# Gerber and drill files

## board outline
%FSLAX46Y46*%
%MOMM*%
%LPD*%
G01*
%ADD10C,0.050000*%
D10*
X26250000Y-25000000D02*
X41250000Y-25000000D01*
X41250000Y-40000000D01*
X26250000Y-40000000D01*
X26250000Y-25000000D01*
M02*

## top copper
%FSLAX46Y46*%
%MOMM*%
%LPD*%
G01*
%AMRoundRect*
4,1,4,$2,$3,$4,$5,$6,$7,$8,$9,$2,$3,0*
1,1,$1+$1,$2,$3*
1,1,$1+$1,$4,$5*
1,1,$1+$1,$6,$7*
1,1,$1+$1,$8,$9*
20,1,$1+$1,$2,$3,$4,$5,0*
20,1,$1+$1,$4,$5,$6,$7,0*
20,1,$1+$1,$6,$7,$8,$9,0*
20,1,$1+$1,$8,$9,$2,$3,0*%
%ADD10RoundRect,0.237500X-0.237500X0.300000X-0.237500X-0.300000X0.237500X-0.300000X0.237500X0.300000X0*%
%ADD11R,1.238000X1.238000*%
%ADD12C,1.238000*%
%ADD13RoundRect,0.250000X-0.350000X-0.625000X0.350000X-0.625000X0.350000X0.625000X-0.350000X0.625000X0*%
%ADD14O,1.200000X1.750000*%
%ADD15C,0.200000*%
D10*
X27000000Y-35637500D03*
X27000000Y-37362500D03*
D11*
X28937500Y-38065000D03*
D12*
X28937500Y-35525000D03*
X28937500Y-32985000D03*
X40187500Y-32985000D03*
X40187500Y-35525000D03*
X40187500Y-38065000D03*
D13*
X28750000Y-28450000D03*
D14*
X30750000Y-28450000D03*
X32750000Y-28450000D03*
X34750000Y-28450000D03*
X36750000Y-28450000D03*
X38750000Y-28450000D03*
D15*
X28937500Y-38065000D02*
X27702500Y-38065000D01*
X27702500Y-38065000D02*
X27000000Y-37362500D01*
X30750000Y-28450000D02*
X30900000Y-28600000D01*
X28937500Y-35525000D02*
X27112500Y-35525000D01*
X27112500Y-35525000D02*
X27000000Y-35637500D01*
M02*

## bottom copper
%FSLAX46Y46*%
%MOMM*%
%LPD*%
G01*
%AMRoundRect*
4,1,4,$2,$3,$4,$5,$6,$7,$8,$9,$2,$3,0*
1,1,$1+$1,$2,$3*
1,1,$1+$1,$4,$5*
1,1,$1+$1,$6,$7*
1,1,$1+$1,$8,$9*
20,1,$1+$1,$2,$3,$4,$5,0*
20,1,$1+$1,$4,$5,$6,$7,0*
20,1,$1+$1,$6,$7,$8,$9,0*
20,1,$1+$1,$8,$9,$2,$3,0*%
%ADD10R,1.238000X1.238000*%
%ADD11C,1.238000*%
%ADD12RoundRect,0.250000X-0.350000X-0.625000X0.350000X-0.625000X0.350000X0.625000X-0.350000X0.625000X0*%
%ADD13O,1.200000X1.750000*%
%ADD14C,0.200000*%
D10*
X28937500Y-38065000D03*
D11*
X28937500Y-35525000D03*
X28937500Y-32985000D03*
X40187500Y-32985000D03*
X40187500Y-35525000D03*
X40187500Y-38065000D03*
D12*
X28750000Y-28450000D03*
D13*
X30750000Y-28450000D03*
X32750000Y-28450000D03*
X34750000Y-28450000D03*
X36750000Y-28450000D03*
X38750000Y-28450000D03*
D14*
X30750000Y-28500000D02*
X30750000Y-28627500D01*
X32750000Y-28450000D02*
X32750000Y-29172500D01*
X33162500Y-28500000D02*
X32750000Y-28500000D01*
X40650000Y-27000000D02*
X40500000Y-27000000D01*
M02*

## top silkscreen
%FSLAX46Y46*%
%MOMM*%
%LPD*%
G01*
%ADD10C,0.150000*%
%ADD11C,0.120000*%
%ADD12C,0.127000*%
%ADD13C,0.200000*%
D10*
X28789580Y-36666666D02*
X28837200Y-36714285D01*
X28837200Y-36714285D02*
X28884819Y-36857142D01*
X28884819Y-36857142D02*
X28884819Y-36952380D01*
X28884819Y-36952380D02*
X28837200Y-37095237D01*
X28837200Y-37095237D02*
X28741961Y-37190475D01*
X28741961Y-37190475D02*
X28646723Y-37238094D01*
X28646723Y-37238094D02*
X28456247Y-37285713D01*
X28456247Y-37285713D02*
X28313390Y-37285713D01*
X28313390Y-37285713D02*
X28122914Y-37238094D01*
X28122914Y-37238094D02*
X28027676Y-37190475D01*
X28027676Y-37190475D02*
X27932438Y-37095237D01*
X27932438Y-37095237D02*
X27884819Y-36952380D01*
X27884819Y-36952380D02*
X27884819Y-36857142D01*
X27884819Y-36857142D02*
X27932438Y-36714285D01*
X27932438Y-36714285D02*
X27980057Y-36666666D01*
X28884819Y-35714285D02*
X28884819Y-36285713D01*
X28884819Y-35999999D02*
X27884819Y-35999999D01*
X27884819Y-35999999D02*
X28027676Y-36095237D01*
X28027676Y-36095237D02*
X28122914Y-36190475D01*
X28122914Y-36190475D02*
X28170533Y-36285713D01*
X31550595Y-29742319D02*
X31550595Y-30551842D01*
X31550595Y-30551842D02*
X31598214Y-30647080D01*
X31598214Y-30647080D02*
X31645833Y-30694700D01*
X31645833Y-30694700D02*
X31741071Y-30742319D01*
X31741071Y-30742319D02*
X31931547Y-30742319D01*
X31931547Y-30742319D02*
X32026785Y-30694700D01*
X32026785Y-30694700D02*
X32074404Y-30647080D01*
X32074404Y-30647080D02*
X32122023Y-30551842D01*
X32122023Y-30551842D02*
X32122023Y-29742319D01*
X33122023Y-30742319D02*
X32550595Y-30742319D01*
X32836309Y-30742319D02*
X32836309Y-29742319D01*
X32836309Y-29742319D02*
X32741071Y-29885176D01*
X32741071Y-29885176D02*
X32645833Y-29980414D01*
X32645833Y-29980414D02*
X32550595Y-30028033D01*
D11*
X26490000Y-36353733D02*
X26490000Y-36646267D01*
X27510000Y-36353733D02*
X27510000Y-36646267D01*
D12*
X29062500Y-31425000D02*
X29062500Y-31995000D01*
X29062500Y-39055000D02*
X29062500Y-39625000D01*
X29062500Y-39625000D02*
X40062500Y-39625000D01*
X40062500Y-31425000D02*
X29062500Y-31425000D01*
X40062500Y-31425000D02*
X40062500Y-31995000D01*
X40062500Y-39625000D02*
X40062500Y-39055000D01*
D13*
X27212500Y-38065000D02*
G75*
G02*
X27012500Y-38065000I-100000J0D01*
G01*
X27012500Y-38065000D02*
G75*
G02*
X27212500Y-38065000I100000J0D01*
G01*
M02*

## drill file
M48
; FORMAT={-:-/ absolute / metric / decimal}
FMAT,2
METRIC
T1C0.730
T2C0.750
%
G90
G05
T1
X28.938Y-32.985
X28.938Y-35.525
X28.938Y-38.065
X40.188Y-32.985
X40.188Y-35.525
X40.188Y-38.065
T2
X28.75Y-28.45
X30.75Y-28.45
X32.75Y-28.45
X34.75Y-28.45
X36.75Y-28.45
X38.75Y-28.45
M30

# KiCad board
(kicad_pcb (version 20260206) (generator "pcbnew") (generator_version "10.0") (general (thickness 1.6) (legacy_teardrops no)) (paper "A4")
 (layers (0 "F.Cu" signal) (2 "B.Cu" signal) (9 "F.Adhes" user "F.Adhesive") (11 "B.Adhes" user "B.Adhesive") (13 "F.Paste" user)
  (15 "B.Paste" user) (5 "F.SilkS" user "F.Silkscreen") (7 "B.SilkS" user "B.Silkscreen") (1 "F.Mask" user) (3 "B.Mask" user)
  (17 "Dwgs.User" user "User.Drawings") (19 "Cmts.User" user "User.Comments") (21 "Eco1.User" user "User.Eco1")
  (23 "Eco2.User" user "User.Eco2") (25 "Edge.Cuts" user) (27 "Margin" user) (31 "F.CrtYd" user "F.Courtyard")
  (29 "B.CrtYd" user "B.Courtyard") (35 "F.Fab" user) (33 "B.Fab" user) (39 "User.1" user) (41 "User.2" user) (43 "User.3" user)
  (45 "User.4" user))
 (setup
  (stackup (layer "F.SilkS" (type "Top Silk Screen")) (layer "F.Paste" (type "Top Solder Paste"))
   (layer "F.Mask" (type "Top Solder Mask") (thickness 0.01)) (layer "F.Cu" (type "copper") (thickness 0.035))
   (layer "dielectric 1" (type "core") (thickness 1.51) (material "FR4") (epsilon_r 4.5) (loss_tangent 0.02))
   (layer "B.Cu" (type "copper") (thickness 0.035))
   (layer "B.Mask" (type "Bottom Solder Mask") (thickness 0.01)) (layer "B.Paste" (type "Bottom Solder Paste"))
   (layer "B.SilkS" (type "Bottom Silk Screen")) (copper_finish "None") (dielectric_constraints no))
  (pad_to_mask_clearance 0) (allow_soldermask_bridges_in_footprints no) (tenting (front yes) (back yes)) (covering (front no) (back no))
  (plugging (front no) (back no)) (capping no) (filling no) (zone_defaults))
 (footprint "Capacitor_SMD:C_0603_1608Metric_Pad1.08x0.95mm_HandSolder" (layer "F.Cu") (at 27 36.5 -90)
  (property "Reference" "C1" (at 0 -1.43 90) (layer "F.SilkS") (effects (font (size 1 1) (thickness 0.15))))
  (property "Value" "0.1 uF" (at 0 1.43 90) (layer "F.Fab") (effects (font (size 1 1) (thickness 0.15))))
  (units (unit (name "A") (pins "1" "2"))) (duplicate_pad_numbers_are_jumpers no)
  (fp_line (start -0.146267 0.51) (end 0.146267 0.51) (stroke (width 0.12) (type solid)) (layer "F.SilkS"))
  (fp_line (start -0.146267 -0.51) (end 0.146267 -0.51) (stroke (width 0.12) (type solid)) (layer "F.SilkS"))
  (pad "1" smd roundrect (at -0.8625 0 270) (size 1.075 0.95) (layers "F.Cu" "F.Mask" "F.Paste") (roundrect_rratio 0.25)
   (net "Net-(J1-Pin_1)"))
  (pad "2" smd roundrect (at 0.8625 0 270) (size 1.075 0.95) (layers "F.Cu" "F.Mask" "F.Paste") (roundrect_rratio 0.25)
   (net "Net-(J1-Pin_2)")))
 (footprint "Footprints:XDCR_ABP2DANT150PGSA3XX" (layer "F.Cu") (at 34.5625 35.525)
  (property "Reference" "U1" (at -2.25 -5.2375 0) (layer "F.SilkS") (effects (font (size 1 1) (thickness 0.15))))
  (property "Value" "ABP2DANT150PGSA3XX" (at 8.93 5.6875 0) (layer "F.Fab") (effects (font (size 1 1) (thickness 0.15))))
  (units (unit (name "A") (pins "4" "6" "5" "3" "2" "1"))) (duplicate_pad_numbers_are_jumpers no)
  (fp_line (start -5.5 -4.1) (end -5.5 -3.53) (stroke (width 0.127) (type solid)) (layer "F.SilkS"))
  (fp_line (start -5.5 3.53) (end -5.5 4.1) (stroke (width 0.127) (type solid)) (layer "F.SilkS"))
  (fp_line (start -5.5 4.1) (end 5.5 4.1) (stroke (width 0.127) (type solid)) (layer "F.SilkS"))
  (fp_line (start 5.5 -4.1) (end -5.5 -4.1) (stroke (width 0.127) (type solid)) (layer "F.SilkS"))
  (fp_line (start 5.5 -4.1) (end 5.5 -3.53) (stroke (width 0.127) (type solid)) (layer "F.SilkS"))
  (fp_line (start 5.5 4.1) (end 5.5 3.53) (stroke (width 0.127) (type solid)) (layer "F.SilkS"))
  (fp_circle (center -7.45 2.54) (end -7.35 2.54) (stroke (width 0.2) (type solid)) (fill no) (layer "F.SilkS"))
  (pad "1" thru_hole rect (at -5.625 2.54) (size 1.238 1.238) (drill 0.73) (layers "*.Cu" "*.Mask") (remove_unused_layers no)
   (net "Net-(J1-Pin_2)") (solder_mask_margin 0.102))
  (pad "2" thru_hole circle (at -5.625 0) (size 1.238 1.238) (drill 0.73) (layers "*.Cu" "*.Mask") (remove_unused_layers no)
   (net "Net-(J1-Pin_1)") (solder_mask_margin 0.102))
  (pad "3" thru_hole circle (at -5.625 -2.54) (size 1.238 1.238) (drill 0.73) (layers "*.Cu" "*.Mask") (remove_unused_layers no)
   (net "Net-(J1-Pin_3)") (solder_mask_margin 0.102))
  (pad "4" thru_hole circle (at 5.625 -2.54) (size 1.238 1.238) (drill 0.73) (layers "*.Cu" "*.Mask") (remove_unused_layers no)
   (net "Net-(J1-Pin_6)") (solder_mask_margin 0.102))
  (pad "5" thru_hole circle (at 5.625 0) (size 1.238 1.238) (drill 0.73) (layers "*.Cu" "*.Mask") (remove_unused_layers no)
   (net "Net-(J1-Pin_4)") (solder_mask_margin 0.102))
  (pad "6" thru_hole circle (at 5.625 2.54) (size 1.238 1.238) (drill 0.73) (layers "*.Cu" "*.Mask") (remove_unused_layers no)
   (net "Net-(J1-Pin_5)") (solder_mask_margin 0.102)))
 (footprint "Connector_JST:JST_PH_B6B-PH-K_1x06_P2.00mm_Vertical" (layer "B.Cu") (at 28.75 28.45)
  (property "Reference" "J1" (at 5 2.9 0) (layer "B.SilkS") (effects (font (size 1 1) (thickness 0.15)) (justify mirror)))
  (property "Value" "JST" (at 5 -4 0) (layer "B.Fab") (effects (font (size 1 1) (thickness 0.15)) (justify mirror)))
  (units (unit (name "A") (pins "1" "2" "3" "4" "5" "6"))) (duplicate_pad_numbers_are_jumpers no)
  (pad "1" thru_hole roundrect (at 0 0) (size 1.2 1.75) (drill 0.75) (layers "*.Cu" "*.Mask") (remove_unused_layers no)
   (roundrect_rratio 0.208333) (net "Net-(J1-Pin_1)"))
  (pad "2" thru_hole oval (at 2 0) (size 1.2 1.75) (drill 0.75) (layers "*.Cu" "*.Mask") (remove_unused_layers no) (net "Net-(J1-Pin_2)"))
  (pad "3" thru_hole oval (at 4 0) (size 1.2 1.75) (drill 0.75) (layers "*.Cu" "*.Mask") (remove_unused_layers no) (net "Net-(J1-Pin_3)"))
  (pad "4" thru_hole oval (at 6 0) (size 1.2 1.75) (drill 0.75) (layers "*.Cu" "*.Mask") (remove_unused_layers no) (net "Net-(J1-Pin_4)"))
  (pad "5" thru_hole oval (at 8 0) (size 1.2 1.75) (drill 0.75) (layers "*.Cu" "*.Mask") (remove_unused_layers no) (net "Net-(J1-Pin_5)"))
  (pad "6" thru_hole oval (at 10 0) (size 1.2 1.75) (drill 0.75) (layers "*.Cu" "*.Mask") (remove_unused_layers no) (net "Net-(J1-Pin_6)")))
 (gr_rect (start 26.25 25) (end 41.25 40) (stroke (width 0.05) (type default)) (fill no) (layer "Edge.Cuts"))
 (segment (start 28.9375 38.065) (end 27.7025 38.065) (width 0.2) (layer "F.Cu") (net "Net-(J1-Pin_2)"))
 (segment (start 27.7025 38.065) (end 27 37.3625) (width 0.2) (layer "F.Cu") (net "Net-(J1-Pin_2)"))
 (segment (start 30.75 28.45) (end 30.9 28.6) (width 0.2) (layer "F.Cu") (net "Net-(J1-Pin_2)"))
 (segment (start 30.75 28.5) (end 30.75 28.6275) (width 0.2) (layer "B.Cu") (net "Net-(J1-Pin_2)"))
 (segment (start 28.9375 35.525) (end 27.1125 35.525) (width 0.2) (layer "F.Cu") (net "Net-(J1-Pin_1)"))
 (segment (start 27.1125 35.525) (end 27 35.6375) (width 0.2) (layer "F.Cu") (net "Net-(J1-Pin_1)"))
 (segment (start 32.75 28.45) (end 32.75 29.1725) (width 0.2) (layer "B.Cu") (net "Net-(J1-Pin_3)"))
 (segment (start 33.1625 28.5) (end 32.75 28.5) (width 0.2) (layer "B.Cu") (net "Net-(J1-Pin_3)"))
 (segment (start 40.65 27) (end 40.5 27) (width 0.2) (layer "B.Cu") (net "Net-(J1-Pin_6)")))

